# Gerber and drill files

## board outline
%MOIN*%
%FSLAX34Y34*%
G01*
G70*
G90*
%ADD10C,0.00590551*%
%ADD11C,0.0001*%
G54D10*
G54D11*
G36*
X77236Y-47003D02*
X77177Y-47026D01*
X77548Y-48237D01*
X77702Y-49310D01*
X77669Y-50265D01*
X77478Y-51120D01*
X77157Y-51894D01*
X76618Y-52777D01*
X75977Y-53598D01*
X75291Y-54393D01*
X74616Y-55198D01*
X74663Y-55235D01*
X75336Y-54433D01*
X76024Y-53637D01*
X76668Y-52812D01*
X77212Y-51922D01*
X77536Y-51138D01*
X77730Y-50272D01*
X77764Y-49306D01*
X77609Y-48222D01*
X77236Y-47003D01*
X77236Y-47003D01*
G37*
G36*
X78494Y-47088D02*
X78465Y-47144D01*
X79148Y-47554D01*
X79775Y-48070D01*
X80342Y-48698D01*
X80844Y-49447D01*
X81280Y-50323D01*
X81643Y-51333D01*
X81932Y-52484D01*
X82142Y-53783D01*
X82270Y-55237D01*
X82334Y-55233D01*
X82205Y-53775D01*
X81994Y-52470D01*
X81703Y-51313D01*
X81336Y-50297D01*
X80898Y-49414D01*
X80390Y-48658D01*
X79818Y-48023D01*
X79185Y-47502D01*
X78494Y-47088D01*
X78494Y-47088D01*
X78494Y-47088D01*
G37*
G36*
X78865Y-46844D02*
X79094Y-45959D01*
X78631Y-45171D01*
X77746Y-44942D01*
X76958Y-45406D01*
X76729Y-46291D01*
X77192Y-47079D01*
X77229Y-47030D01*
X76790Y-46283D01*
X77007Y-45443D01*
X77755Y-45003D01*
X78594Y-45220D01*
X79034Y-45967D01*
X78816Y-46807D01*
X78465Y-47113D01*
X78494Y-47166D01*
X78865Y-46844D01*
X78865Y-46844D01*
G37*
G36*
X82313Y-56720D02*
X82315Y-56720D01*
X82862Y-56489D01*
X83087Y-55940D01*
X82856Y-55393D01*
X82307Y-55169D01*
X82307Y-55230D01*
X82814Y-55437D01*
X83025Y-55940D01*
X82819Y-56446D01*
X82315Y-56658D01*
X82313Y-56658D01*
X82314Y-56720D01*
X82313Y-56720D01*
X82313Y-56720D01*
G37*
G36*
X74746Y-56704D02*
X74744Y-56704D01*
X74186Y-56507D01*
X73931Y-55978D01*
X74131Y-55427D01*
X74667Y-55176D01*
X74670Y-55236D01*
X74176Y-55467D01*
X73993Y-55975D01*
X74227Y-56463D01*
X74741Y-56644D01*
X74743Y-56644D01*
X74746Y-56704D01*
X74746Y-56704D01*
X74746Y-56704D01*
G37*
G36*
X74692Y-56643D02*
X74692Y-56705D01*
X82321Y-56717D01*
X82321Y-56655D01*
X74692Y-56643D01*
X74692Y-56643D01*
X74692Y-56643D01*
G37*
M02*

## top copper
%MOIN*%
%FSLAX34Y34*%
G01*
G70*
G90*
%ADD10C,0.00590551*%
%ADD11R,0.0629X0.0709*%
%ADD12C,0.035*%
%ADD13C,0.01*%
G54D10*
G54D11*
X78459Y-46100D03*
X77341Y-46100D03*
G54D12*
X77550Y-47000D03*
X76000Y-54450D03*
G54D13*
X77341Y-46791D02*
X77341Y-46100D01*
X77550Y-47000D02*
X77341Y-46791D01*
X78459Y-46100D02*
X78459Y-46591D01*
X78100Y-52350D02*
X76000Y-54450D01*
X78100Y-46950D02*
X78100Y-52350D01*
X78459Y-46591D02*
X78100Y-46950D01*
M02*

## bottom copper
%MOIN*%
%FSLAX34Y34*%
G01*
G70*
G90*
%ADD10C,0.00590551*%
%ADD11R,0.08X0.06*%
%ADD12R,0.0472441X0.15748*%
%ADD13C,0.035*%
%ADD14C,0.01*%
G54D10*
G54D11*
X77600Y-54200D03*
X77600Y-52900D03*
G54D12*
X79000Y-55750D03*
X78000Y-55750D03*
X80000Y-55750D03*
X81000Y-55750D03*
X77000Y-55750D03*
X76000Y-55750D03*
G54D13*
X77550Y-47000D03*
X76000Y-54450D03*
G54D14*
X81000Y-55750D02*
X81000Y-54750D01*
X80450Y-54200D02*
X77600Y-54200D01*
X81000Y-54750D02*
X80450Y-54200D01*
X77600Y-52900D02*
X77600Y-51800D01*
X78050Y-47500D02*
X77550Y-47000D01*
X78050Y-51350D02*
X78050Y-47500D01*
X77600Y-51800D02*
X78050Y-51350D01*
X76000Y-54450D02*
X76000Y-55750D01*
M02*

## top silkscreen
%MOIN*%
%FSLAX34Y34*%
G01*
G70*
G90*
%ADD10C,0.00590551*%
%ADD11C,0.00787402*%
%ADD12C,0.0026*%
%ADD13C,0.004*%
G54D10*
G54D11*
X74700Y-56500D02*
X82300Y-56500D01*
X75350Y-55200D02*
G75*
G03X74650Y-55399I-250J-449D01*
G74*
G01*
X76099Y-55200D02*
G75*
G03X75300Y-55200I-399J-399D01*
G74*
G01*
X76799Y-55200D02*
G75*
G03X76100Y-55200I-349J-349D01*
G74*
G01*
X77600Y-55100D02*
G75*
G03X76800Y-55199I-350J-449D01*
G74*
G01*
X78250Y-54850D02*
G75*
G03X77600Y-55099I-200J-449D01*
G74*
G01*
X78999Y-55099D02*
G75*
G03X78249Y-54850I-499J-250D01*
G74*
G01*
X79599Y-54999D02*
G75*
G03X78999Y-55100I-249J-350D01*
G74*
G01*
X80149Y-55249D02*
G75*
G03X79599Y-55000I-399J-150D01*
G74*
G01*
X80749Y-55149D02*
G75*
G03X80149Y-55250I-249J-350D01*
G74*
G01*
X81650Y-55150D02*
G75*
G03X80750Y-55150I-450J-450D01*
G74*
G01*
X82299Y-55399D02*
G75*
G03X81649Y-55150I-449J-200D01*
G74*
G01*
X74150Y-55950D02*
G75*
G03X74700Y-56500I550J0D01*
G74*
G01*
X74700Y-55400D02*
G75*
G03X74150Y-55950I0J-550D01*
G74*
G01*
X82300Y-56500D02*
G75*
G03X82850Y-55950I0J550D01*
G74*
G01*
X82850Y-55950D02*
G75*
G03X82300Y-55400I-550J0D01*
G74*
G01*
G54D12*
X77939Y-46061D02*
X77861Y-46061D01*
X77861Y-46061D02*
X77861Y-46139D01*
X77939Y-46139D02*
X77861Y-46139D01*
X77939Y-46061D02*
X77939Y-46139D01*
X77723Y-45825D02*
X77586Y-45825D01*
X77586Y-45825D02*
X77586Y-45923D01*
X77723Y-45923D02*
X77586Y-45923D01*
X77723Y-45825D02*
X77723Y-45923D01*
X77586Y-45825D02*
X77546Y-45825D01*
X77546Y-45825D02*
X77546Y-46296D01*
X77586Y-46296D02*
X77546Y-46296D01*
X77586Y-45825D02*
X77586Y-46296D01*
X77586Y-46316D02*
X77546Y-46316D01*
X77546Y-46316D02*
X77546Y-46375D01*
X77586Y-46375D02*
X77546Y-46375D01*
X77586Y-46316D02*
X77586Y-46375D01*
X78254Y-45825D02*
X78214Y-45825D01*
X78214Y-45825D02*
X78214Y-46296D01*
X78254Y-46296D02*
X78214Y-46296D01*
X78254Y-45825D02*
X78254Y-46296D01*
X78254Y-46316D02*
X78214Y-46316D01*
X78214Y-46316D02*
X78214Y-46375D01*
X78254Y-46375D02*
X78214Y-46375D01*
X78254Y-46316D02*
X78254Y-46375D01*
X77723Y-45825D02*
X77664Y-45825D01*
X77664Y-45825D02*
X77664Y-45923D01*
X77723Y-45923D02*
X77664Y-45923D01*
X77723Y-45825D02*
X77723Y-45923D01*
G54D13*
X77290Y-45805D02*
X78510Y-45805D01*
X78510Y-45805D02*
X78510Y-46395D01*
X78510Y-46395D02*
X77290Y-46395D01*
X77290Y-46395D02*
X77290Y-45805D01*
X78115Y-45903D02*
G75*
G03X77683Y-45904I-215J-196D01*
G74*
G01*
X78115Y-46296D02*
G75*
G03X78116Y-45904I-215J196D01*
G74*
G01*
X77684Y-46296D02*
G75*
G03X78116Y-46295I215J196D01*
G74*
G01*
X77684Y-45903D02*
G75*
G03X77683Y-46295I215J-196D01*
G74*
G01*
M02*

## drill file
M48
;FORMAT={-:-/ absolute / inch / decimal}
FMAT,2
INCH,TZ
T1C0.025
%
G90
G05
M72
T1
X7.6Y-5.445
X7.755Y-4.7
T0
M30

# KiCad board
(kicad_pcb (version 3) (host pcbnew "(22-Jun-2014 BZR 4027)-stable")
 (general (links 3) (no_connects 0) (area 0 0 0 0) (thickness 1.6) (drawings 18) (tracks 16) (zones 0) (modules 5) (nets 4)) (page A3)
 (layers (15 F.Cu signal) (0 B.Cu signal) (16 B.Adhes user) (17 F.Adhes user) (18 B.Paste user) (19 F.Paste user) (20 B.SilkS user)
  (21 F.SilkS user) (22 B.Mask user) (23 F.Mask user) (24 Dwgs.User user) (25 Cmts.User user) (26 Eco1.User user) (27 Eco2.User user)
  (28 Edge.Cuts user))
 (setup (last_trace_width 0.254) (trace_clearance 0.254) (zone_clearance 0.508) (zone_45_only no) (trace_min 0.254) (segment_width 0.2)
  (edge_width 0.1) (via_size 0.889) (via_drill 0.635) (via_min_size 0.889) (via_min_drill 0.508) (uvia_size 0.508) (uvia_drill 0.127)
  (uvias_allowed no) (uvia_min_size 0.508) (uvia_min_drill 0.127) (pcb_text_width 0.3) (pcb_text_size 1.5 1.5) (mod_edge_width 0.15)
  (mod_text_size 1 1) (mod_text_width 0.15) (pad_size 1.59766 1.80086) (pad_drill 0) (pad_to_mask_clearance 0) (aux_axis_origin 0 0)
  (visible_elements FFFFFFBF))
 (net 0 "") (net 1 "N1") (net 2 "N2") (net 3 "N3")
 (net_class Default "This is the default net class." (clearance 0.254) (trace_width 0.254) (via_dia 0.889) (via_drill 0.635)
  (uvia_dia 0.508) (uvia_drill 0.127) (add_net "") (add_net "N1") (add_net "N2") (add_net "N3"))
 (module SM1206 (layer B.Cu) (at 197.104 136.017 90)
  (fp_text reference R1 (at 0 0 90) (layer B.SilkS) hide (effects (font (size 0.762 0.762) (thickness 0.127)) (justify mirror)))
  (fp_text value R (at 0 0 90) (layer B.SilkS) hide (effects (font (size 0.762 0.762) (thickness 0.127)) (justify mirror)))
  (pad 1 smd rect (at -1.651 0 90) (size 1.524 2.032) (layers B.Cu B.Paste B.Mask) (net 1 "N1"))
  (pad 2 smd rect (at 1.651 0 90) (size 1.524 2.032) (layers B.Cu B.Paste B.Mask) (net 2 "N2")))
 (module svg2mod (layer F.Cu) (at 199.39 128.905)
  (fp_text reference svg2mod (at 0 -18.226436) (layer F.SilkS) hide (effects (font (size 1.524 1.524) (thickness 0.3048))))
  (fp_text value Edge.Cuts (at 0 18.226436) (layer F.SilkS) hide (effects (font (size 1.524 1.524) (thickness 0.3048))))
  (fp_poly
   (pts (xy -3.209801 -9.515198) (xy -3.359404 -9.457433) (xy -2.417162 -6.382811) (xy -2.024726 -3.656767) (xy -2.108415 -1.231527)
    (xy -2.594552 0.940684) (xy -3.409456 2.90764) (xy -4.779605 5.149717) (xy -6.407762 7.235427) (xy -8.150723 9.254938)
    (xy -9.865284 11.29842) (xy -9.745641 11.39267) (xy -8.034736 9.355289) (xy -6.288756 7.334351) (xy -4.652556 5.238653)
    (xy -3.270989 2.976987) (xy -2.447368 0.987114) (xy -1.95541 -1.212272) (xy -1.869144 -3.665941) (xy -2.262598 -6.418661)
    (xy -3.209801 -9.515198))
   (layer Edge.Cuts) (width 0.00254))
  (fp_poly
   (pts (xy -0.014213 -9.300715) (xy -0.088305 -9.157233) (xy 1.647664 -8.116827) (xy 3.239948 -6.806913) (xy 4.679206 -5.209767)
    (xy 5.956094 -3.307662) (xy 7.061267 -1.082874) (xy 7.985382 1.482323) (xy 8.719097 4.405656) (xy 9.253066 7.704849)
    (xy 9.577948 11.397629) (xy 9.738639 11.388316) (xy 9.412364 7.684043) (xy 8.875243 4.370861) (xy 8.13649 1.431748)
    (xy 7.205323 -1.150319) (xy 6.090955 -3.392361) (xy 4.802602 -5.311401) (xy 3.349479 -6.924462) (xy 1.740803 -8.248564)
    (xy -0.014213 -9.300732) (xy -0.014213 -9.300715))
   (layer Edge.Cuts) (width 0.00254))
  (fp_poly
   (pts (xy 0.92723 -9.919482) (xy 1.510311 -12.168182) (xy 0.334916 -14.170423) (xy -1.913306 -14.750093) (xy -3.915066 -13.571285)
    (xy -4.496679 -11.324531) (xy -3.31982 -9.324236) (xy -3.225882 -9.448794) (xy -4.34315 -11.346049) (xy -3.790507 -13.477347)
    (xy -1.891787 -14.596562) (xy 0.240984 -14.045864) (xy 1.356778 -12.146664) (xy 0.802671 -10.013419) (xy -0.087678 -9.237664)
    (xy -0.01296 -9.101932) (xy 0.92723 -9.919482))
   (layer Edge.Cuts) (width 0.00254))
  (fp_poly
   (pts (xy 9.687235 15.164161) (xy 9.692146 15.16413) (xy 11.081337 14.579363) (xy 11.651231 13.183991) (xy 11.066463 11.794797)
    (xy 9.671092 11.224903) (xy 9.672221 11.380913) (xy 10.957715 11.905005) (xy 11.495518 13.18483) (xy 10.971426 14.47032)
    (xy 9.691604 15.008123) (xy 9.686694 15.008149) (xy 9.687822 15.164161) (xy 9.687235 15.164161))
   (layer Edge.Cuts) (width 0.00254))
  (fp_poly
   (pts (xy -9.533213 15.125025) (xy -9.538123 15.125223) (xy -10.957366 14.624453) (xy -11.603104 13.280664) (xy -11.095579 11.88032)
    (xy -9.733653 11.24318) (xy -9.72592 11.396926) (xy -10.980658 11.98299) (xy -11.447292 13.273024) (xy -10.853327 14.511053)
    (xy -9.545876 14.971474) (xy -9.540965 14.971285) (xy -9.533204 15.125025) (xy -9.533213 15.125025))
   (layer Edge.Cuts) (width 0.00254))
  (fp_poly
   (pts (xy -9.671798 14.969809) (xy -9.67208 15.125895) (xy 9.706266 15.1571) (xy 9.706548 15.001014) (xy -9.671795 14.969809)
    (xy -9.671798 14.969809))
   (layer Edge.Cuts) (width 0.00254)))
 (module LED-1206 (layer F.Cu) (at 197.866 117.094 180)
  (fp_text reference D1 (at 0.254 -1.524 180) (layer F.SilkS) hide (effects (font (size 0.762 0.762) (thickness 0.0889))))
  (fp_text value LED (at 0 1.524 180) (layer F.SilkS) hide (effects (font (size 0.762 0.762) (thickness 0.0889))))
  (fp_line (start -0.09906 0.09906) (end 0.09906 0.09906) (layer F.SilkS) (width 0.06604))
  (fp_line (start 0.09906 0.09906) (end 0.09906 -0.09906) (layer F.SilkS) (width 0.06604))
  (fp_line (start -0.09906 -0.09906) (end 0.09906 -0.09906) (layer F.SilkS) (width 0.06604))
  (fp_line (start -0.09906 0.09906) (end -0.09906 -0.09906) (layer F.SilkS) (width 0.06604))
  (fp_line (start 0.44958 0.6985) (end 0.79756 0.6985) (layer F.SilkS) (width 0.06604))
  (fp_line (start 0.79756 0.6985) (end 0.79756 0.44958) (layer F.SilkS) (width 0.06604))
  (fp_line (start 0.44958 0.44958) (end 0.79756 0.44958) (layer F.SilkS) (width 0.06604))
  (fp_line (start 0.44958 0.6985) (end 0.44958 0.44958) (layer F.SilkS) (width 0.06604))
  (fp_line (start 0.79756 0.6985) (end 0.89916 0.6985) (layer F.SilkS) (width 0.06604))
  (fp_line (start 0.89916 0.6985) (end 0.89916 -0.49784) (layer F.SilkS) (width 0.06604))
  (fp_line (start 0.79756 -0.49784) (end 0.89916 -0.49784) (layer F.SilkS) (width 0.06604))
  (fp_line (start 0.79756 0.6985) (end 0.79756 -0.49784) (layer F.SilkS) (width 0.06604))
  (fp_line (start 0.79756 -0.54864) (end 0.89916 -0.54864) (layer F.SilkS) (width 0.06604))
  (fp_line (start 0.89916 -0.54864) (end 0.89916 -0.6985) (layer F.SilkS) (width 0.06604))
  (fp_line (start 0.79756 -0.6985) (end 0.89916 -0.6985) (layer F.SilkS) (width 0.06604))
  (fp_line (start 0.79756 -0.54864) (end 0.79756 -0.6985) (layer F.SilkS) (width 0.06604))
  (fp_line (start -0.89916 0.6985) (end -0.79756 0.6985) (layer F.SilkS) (width 0.06604))
  (fp_line (start -0.79756 0.6985) (end -0.79756 -0.49784) (layer F.SilkS) (width 0.06604))
  (fp_line (start -0.89916 -0.49784) (end -0.79756 -0.49784) (layer F.SilkS) (width 0.06604))
  (fp_line (start -0.89916 0.6985) (end -0.89916 -0.49784) (layer F.SilkS) (width 0.06604))
  (fp_line (start -0.89916 -0.54864) (end -0.79756 -0.54864) (layer F.SilkS) (width 0.06604))
  (fp_line (start -0.79756 -0.54864) (end -0.79756 -0.6985) (layer F.SilkS) (width 0.06604))
  (fp_line (start -0.89916 -0.6985) (end -0.79756 -0.6985) (layer F.SilkS) (width 0.06604))
  (fp_line (start -0.89916 -0.54864) (end -0.89916 -0.6985) (layer F.SilkS) (width 0.06604))
  (fp_line (start 0.44958 0.6985) (end 0.59944 0.6985) (layer F.SilkS) (width 0.06604))
  (fp_line (start 0.59944 0.6985) (end 0.59944 0.44958) (layer F.SilkS) (width 0.06604))
  (fp_line (start 0.44958 0.44958) (end 0.59944 0.44958) (layer F.SilkS) (width 0.06604))
  (fp_line (start 0.44958 0.6985) (end 0.44958 0.44958) (layer F.SilkS) (width 0.06604))
  (fp_line (start 1.5494 0.7493) (end -1.5494 0.7493) (layer F.SilkS) (width 0.1016))
  (fp_line (start -1.5494 0.7493) (end -1.5494 -0.7493) (layer F.SilkS) (width 0.1016))
  (fp_line (start -1.5494 -0.7493) (end 1.5494 -0.7493) (layer F.SilkS) (width 0.1016))
  (fp_line (start 1.5494 -0.7493) (end 1.5494 0.7493) (layer F.SilkS) (width 0.1016))
  (fp_arc (start 0 0) (end 0.54864 0.49784) (angle 95.4) (layer F.SilkS) (width 0.1016))
  (fp_arc (start 0 0) (end -0.54864 0.49784) (angle 84.5) (layer F.SilkS) (width 0.1016))
  (fp_arc (start 0 0) (end -0.54864 -0.49784) (angle 95.4) (layer F.SilkS) (width 0.1016))
  (fp_arc (start 0 0) (end 0.54864 -0.49784) (angle 84.5) (layer F.SilkS) (width 0.1016))
  (pad 1 smd rect (at -1.41986 0 180) (size 1.59766 1.80086) (layers F.Cu F.Paste F.Mask) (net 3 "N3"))
  (pad 2 smd rect (at 1.41986 0 180) (size 1.59766 1.80086) (layers F.Cu F.Paste F.Mask) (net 2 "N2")))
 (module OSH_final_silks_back (layer F.Cu) (at 203.073 135.255)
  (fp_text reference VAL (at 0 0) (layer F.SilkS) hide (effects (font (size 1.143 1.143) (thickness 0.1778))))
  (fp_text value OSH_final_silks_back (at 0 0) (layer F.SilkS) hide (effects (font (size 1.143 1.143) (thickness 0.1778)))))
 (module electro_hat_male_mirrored (layer B.Cu) (at 199.39 141.605)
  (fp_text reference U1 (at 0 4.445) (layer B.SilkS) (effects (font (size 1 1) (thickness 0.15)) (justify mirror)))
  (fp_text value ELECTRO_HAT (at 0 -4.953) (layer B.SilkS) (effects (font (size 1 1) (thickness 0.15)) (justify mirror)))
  (pad 3 smd rect (at 1.27 0) (size 1.2 4) (layers B.Cu B.Paste B.Mask))
  (pad 4 smd rect (at -1.27 0) (size 1.2 4) (layers B.Cu B.Paste B.Mask))
  (pad 2 smd rect (at 3.81 0) (size 1.2 4) (layers B.Cu B.Paste B.Mask))
  (pad 1 smd rect (at 6.35 0) (size 1.2 4) (layers B.Cu B.Paste B.Mask) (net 1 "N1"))
  (pad 5 smd rect (at -3.81 0) (size 1.2 4) (layers B.Cu B.Paste B.Mask))
  (pad 6 smd rect (at -6.35 0) (size 1.2 4) (layers B.Cu B.Paste B.Mask) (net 3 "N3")))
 (gr_line (start 189.738 143.51) (end 209.042 143.51) (angle 90) (layer F.SilkS) (width 0.2))
 (gr_arc (start 190.754 141.351) (end 189.611 140.716) (angle 90) (layer F.SilkS) (width 0.2))
 (gr_arc (start 192.278 141.224) (end 191.262 140.208) (angle 90) (layer F.SilkS) (width 0.2))
 (gr_arc (start 194.183 141.097) (end 193.294 140.208) (angle 90) (layer F.SilkS) (width 0.2))
 (gr_arc (start 196.215 141.097) (end 195.072 140.208) (angle 90) (layer F.SilkS) (width 0.2))
 (gr_arc (start 198.247 140.462) (end 197.104 139.954) (angle 90) (layer F.SilkS) (width 0.2))
 (gr_arc (start 199.39 140.589) (end 198.755 139.319) (angle 90) (layer F.SilkS) (width 0.2))
 (gr_arc (start 201.549 140.589) (end 200.66 139.954) (angle 90) (layer F.SilkS) (width 0.2))
 (gr_arc (start 202.565 140.716) (end 202.184 139.7) (angle 90) (layer F.SilkS) (width 0.2))
 (gr_arc (start 204.47 140.97) (end 203.581 140.335) (angle 90) (layer F.SilkS) (width 0.2))
 (gr_arc (start 206.248 141.224) (end 205.105 140.081) (angle 90) (layer F.SilkS) (width 0.2))
 (gr_arc (start 207.899 141.224) (end 207.391 140.081) (angle 90) (layer F.SilkS) (width 0.2))
 (gr_arc (start 189.738 142.113) (end 189.738 143.51) (angle 90) (layer F.SilkS) (width 0.2))
 (gr_arc (start 189.738 142.113) (end 188.341 142.113) (angle 90) (layer F.SilkS) (width 0.2))
 (gr_arc (start 209.042 142.113) (end 210.439 142.113) (angle 90) (layer F.SilkS) (width 0.2))
 (gr_arc (start 209.042 142.113) (end 209.042 140.716) (angle 90) (layer F.SilkS) (width 0.2))
 (segment (start 205.74 141.605) (end 205.74 139.065) (width 0.254) (layer B.Cu) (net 1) (status 400000))
 (segment (start 204.343 137.668) (end 197.104 137.668) (width 0.254) (layer B.Cu) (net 1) (status 800000))
 (segment (start 205.74 139.065) (end 204.343 137.668) (width 0.254) (layer B.Cu) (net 1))
 (segment (start 197.104 134.366) (end 197.104 131.572) (width 0.254) (layer B.Cu) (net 2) (status 400000))
 (segment (start 196.44614 118.84914) (end 196.44614 117.094) (width 0.254) (layer F.Cu) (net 2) (status 800000))
 (segment (start 196.977 119.38) (end 196.44614 118.84914) (width 0.254) (layer F.Cu) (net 2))
 (via (at 196.977 119.38) (size 0.889) (layers F.Cu B.Cu) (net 2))
 (segment (start 198.247 120.65) (end 196.977 119.38) (width 0.254) (layer B.Cu) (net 2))
 (segment (start 198.247 130.429) (end 198.247 120.65) (width 0.254) (layer B.Cu) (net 2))
 (segment (start 197.104 131.572) (end 198.247 130.429) (width 0.254) (layer B.Cu) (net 2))
 (segment (start 199.28586 117.094) (end 199.28586 118.34114) (width 0.254) (layer F.Cu) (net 3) (status 400000))
 (segment (start 193.04 138.303) (end 193.04 141.605) (width 0.254) (layer B.Cu) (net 3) (status 800000))
 (via (at 193.04 138.303) (size 0.889) (layers F.Cu B.Cu) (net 3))
 (segment (start 198.374 132.969) (end 193.04 138.303) (width 0.254) (layer F.Cu) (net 3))
 (segment (start 198.374 119.253) (end 198.374 132.969) (width 0.254) (layer F.Cu) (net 3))
 (segment (start 199.28586 118.34114) (end 198.374 119.253) (width 0.254) (layer F.Cu) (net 3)))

